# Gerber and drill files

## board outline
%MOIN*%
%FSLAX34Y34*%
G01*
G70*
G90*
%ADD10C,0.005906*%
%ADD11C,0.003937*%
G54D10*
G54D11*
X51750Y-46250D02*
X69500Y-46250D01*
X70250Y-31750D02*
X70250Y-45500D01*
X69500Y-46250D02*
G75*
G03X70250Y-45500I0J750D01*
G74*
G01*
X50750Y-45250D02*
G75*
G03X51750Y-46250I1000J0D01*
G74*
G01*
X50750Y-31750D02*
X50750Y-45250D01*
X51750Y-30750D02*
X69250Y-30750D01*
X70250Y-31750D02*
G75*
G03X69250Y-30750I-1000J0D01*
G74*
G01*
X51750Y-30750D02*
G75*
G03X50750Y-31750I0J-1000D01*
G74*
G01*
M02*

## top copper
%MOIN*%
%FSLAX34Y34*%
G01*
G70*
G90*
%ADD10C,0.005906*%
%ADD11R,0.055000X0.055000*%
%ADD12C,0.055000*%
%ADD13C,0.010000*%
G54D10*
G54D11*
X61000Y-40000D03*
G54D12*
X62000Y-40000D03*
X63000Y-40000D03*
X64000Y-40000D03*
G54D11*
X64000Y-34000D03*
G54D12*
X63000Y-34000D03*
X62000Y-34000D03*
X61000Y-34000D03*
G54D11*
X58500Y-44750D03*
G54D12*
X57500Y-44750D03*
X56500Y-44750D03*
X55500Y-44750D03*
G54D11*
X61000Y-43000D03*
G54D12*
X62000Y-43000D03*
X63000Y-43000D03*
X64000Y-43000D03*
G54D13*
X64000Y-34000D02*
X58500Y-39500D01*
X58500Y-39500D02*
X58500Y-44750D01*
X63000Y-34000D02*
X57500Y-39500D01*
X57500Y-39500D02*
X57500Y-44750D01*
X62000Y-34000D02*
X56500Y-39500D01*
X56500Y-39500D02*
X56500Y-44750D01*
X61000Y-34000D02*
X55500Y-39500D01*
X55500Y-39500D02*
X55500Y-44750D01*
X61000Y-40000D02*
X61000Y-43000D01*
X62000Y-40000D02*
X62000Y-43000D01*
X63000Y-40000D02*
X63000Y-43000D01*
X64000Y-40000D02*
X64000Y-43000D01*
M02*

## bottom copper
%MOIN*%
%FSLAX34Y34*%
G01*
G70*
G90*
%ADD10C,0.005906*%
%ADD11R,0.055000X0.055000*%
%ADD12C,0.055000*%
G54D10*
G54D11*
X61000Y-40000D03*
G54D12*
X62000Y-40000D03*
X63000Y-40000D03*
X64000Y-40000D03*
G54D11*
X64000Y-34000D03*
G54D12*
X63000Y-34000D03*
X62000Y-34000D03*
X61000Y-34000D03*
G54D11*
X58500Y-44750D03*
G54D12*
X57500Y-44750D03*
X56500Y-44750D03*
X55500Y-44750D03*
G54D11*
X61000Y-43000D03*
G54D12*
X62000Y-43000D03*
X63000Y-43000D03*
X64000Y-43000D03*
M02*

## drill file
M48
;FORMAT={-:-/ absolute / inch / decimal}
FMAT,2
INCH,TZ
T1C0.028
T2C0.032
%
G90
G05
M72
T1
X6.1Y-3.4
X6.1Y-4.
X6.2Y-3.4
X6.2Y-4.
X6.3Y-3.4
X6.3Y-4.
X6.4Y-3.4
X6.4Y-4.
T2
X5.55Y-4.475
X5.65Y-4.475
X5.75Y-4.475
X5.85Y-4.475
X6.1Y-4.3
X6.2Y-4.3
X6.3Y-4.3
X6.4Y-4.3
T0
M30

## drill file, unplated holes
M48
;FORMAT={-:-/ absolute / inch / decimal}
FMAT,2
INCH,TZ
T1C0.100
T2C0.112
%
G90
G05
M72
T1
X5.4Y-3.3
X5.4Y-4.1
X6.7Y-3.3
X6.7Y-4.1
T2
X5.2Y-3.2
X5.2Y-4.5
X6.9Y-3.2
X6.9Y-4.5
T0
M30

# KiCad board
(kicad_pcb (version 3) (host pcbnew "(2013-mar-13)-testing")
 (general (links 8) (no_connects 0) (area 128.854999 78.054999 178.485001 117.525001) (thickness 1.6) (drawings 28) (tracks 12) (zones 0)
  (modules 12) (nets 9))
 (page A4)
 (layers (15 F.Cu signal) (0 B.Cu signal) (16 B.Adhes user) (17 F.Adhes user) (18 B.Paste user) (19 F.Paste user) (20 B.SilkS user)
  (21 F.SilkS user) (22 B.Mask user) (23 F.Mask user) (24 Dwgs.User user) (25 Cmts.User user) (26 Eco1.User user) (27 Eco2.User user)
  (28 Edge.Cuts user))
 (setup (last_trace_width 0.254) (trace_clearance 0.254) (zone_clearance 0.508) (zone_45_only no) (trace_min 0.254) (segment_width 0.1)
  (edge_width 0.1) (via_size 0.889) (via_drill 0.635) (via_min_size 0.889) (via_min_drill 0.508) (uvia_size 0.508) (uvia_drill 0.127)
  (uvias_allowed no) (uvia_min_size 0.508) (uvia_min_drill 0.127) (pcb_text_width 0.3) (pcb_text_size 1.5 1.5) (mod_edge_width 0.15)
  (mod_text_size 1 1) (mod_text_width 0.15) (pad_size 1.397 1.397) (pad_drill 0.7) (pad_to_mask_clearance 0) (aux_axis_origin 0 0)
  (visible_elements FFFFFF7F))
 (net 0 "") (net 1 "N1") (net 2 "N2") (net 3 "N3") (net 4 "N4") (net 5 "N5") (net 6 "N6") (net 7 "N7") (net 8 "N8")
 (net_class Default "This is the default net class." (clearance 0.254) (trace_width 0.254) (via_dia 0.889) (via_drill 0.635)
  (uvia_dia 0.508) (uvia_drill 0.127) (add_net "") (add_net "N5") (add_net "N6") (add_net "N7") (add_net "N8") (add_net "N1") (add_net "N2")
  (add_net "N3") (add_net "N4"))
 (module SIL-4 (layer F.Cu) (at 158.75 101.6)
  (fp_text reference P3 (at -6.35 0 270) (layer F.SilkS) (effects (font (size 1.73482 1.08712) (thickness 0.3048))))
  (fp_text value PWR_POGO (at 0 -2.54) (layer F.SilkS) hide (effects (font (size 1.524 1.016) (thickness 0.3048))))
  (pad 1 thru_hole rect (at -3.81 0) (size 1.397 1.397) (drill 0.7) (layers *.Cu *.Mask F.SilkS) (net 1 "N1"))
  (pad 2 thru_hole circle (at -1.27 0) (size 1.397 1.397) (drill 0.7) (layers *.Cu *.Mask F.SilkS) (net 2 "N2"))
  (pad 3 thru_hole circle (at 1.27 0) (size 1.397 1.397) (drill 0.7) (layers *.Cu *.Mask F.SilkS) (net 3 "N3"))
  (pad 4 thru_hole circle (at 3.81 0) (size 1.397 1.397) (drill 0.7) (layers *.Cu *.Mask F.SilkS) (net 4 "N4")))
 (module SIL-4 (layer F.Cu) (at 158.75 86.36 180)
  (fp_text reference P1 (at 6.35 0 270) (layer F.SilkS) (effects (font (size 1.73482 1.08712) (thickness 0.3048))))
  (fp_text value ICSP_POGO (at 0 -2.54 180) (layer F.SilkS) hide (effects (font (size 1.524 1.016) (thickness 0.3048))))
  (pad 1 thru_hole rect (at -3.81 0 180) (size 1.397 1.397) (drill 0.7) (layers *.Cu *.Mask F.SilkS) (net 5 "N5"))
  (pad 2 thru_hole circle (at -1.27 0 180) (size 1.397 1.397) (drill 0.7) (layers *.Cu *.Mask F.SilkS) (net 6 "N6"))
  (pad 3 thru_hole circle (at 1.27 0 180) (size 1.397 1.397) (drill 0.7) (layers *.Cu *.Mask F.SilkS) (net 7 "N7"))
  (pad 4 thru_hole circle (at 3.81 0 180) (size 1.397 1.397) (drill 0.7) (layers *.Cu *.Mask F.SilkS) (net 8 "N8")))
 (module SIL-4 (layer F.Cu) (at 144.78 113.665 180)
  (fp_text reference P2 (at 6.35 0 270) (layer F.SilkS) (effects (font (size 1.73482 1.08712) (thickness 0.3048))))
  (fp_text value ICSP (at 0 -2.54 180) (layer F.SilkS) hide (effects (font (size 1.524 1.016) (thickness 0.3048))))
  (pad 1 thru_hole rect (at -3.81 0 180) (size 1.397 1.397) (drill 0.8128) (layers *.Cu *.Mask F.SilkS) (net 5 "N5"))
  (pad 2 thru_hole circle (at -1.27 0 180) (size 1.397 1.397) (drill 0.8128) (layers *.Cu *.Mask F.SilkS) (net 6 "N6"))
  (pad 3 thru_hole circle (at 1.27 0 180) (size 1.397 1.397) (drill 0.8128) (layers *.Cu *.Mask F.SilkS) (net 7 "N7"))
  (pad 4 thru_hole circle (at 3.81 0 180) (size 1.397 1.397) (drill 0.8128) (layers *.Cu *.Mask F.SilkS) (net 8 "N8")))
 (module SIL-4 (layer F.Cu) (at 158.75 109.22)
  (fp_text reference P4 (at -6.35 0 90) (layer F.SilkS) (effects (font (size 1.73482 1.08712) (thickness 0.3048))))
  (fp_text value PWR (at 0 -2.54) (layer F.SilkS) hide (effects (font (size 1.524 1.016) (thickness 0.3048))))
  (pad 1 thru_hole rect (at -3.81 0) (size 1.397 1.397) (drill 0.8128) (layers *.Cu *.Mask F.SilkS) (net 1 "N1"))
  (pad 2 thru_hole circle (at -1.27 0) (size 1.397 1.397) (drill 0.8128) (layers *.Cu *.Mask F.SilkS) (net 2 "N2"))
  (pad 3 thru_hole circle (at 1.27 0) (size 1.397 1.397) (drill 0.8128) (layers *.Cu *.Mask F.SilkS) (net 3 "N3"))
  (pad 4 thru_hole circle (at 3.81 0) (size 1.397 1.397) (drill 0.8128) (layers *.Cu *.Mask F.SilkS) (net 4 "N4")))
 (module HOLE (layer F.Cu) (at 137.16 83.82)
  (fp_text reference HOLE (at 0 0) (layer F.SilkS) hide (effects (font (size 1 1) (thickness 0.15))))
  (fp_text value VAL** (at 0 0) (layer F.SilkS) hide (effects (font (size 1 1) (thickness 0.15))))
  (pad "" np_thru_hole circle (at 0 0) (size 2.54 2.54) (drill 2.54) (layers *.Cu *.Mask F.SilkS)))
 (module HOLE (layer F.Cu) (at 170.18 83.82)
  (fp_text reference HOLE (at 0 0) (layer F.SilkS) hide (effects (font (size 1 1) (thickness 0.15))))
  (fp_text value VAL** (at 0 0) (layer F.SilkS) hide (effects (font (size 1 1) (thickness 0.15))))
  (pad "" np_thru_hole circle (at 0 0) (size 2.54 2.54) (drill 2.54) (layers *.Cu *.Mask F.SilkS)))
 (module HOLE (layer F.Cu) (at 137.16 104.14)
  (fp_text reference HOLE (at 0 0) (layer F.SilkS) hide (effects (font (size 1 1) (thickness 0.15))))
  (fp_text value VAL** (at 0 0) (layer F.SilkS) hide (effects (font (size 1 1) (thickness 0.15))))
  (pad "" np_thru_hole circle (at 0 0) (size 2.54 2.54) (drill 2.54) (layers *.Cu *.Mask F.SilkS)))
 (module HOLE (layer F.Cu) (at 170.18 104.14)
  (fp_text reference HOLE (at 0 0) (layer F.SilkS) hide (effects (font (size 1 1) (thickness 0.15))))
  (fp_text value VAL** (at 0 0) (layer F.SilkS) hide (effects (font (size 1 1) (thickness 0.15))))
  (pad "" np_thru_hole circle (at 0 0) (size 2.54 2.54) (drill 2.54) (layers *.Cu *.Mask F.SilkS)))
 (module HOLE (layer F.Cu) (at 132.08 81.28)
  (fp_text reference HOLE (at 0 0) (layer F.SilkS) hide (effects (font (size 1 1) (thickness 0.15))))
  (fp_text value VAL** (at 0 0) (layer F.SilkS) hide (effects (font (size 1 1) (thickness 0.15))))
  (pad "" np_thru_hole circle (at 0 0) (size 2.85 2.85) (drill 2.85) (layers *.Cu *.Mask F.SilkS)))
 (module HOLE (layer F.Cu) (at 175.26 81.28)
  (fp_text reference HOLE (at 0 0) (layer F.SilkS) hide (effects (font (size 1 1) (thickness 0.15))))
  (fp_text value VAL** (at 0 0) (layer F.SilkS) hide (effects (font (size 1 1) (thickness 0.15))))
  (pad "" np_thru_hole circle (at 0 0) (size 2.85 2.85) (drill 2.85) (layers *.Cu *.Mask F.SilkS)))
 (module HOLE (layer F.Cu) (at 132.08 114.3)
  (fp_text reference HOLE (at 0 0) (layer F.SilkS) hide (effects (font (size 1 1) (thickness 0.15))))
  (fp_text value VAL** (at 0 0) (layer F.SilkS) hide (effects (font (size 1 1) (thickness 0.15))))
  (pad "" np_thru_hole circle (at 0 0) (size 2.85 2.85) (drill 2.85) (layers *.Cu *.Mask F.SilkS)))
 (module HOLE (layer F.Cu) (at 175.26 114.3)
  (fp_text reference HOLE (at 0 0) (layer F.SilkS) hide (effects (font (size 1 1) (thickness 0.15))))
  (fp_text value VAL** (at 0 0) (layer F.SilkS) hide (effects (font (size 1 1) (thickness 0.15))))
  (pad "" np_thru_hole circle (at 0 0) (size 2.85 2.85) (drill 2.85) (layers *.Cu *.Mask F.SilkS)))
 (gr_line (start 131.445 117.475) (end 176.53 117.475) (angle 90) (layer Edge.Cuts) (width 0.1))
 (gr_line (start 178.435 80.645) (end 178.435 115.57) (angle 90) (layer Edge.Cuts) (width 0.1))
 (gr_arc (start 176.53 115.57) (end 178.435 115.57) (angle 90) (layer Edge.Cuts) (width 0.1))
 (gr_arc (start 131.445 114.935) (end 131.445 117.475) (angle 90) (layer Edge.Cuts) (width 0.1))
 (gr_line (start 128.905 80.645) (end 128.905 114.935) (angle 90) (layer Edge.Cuts) (width 0.1))
 (gr_line (start 131.445 78.105) (end 175.895 78.105) (angle 90) (layer Edge.Cuts) (width 0.1))
 (gr_arc (start 175.895 80.645) (end 175.895 78.105) (angle 90) (layer Edge.Cuts) (width 0.1))
 (gr_arc (start 131.445 80.645) (end 128.905 80.645) (angle 90) (layer Edge.Cuts) (width 0.1))
 (segment (start 162.56 86.36) (end 148.59 100.33) (width 0.254) (layer F.Cu) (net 5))
 (segment (start 148.59 100.33) (end 148.59 113.665) (width 0.254) (layer F.Cu) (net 5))
 (segment (start 160.02 86.36) (end 146.05 100.33) (width 0.254) (layer F.Cu) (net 6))
 (segment (start 146.05 100.33) (end 146.05 113.665) (width 0.254) (layer F.Cu) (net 6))
 (segment (start 157.48 86.36) (end 143.51 100.33) (width 0.254) (layer F.Cu) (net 7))
 (segment (start 143.51 100.33) (end 143.51 113.665) (width 0.254) (layer F.Cu) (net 7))
 (segment (start 154.94 86.36) (end 140.97 100.33) (width 0.254) (layer F.Cu) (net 8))
 (segment (start 140.97 100.33) (end 140.97 113.665) (width 0.254) (layer F.Cu) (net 8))
 (segment (start 154.94 101.6) (end 154.94 109.22) (width 0.254) (layer F.Cu) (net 1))
 (segment (start 157.48 101.6) (end 157.48 109.22) (width 0.254) (layer F.Cu) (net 2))
 (segment (start 160.02 101.6) (end 160.02 109.22) (width 0.254) (layer F.Cu) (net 3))
 (segment (start 162.56 101.6) (end 162.56 109.22) (width 0.254) (layer F.Cu) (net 4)))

